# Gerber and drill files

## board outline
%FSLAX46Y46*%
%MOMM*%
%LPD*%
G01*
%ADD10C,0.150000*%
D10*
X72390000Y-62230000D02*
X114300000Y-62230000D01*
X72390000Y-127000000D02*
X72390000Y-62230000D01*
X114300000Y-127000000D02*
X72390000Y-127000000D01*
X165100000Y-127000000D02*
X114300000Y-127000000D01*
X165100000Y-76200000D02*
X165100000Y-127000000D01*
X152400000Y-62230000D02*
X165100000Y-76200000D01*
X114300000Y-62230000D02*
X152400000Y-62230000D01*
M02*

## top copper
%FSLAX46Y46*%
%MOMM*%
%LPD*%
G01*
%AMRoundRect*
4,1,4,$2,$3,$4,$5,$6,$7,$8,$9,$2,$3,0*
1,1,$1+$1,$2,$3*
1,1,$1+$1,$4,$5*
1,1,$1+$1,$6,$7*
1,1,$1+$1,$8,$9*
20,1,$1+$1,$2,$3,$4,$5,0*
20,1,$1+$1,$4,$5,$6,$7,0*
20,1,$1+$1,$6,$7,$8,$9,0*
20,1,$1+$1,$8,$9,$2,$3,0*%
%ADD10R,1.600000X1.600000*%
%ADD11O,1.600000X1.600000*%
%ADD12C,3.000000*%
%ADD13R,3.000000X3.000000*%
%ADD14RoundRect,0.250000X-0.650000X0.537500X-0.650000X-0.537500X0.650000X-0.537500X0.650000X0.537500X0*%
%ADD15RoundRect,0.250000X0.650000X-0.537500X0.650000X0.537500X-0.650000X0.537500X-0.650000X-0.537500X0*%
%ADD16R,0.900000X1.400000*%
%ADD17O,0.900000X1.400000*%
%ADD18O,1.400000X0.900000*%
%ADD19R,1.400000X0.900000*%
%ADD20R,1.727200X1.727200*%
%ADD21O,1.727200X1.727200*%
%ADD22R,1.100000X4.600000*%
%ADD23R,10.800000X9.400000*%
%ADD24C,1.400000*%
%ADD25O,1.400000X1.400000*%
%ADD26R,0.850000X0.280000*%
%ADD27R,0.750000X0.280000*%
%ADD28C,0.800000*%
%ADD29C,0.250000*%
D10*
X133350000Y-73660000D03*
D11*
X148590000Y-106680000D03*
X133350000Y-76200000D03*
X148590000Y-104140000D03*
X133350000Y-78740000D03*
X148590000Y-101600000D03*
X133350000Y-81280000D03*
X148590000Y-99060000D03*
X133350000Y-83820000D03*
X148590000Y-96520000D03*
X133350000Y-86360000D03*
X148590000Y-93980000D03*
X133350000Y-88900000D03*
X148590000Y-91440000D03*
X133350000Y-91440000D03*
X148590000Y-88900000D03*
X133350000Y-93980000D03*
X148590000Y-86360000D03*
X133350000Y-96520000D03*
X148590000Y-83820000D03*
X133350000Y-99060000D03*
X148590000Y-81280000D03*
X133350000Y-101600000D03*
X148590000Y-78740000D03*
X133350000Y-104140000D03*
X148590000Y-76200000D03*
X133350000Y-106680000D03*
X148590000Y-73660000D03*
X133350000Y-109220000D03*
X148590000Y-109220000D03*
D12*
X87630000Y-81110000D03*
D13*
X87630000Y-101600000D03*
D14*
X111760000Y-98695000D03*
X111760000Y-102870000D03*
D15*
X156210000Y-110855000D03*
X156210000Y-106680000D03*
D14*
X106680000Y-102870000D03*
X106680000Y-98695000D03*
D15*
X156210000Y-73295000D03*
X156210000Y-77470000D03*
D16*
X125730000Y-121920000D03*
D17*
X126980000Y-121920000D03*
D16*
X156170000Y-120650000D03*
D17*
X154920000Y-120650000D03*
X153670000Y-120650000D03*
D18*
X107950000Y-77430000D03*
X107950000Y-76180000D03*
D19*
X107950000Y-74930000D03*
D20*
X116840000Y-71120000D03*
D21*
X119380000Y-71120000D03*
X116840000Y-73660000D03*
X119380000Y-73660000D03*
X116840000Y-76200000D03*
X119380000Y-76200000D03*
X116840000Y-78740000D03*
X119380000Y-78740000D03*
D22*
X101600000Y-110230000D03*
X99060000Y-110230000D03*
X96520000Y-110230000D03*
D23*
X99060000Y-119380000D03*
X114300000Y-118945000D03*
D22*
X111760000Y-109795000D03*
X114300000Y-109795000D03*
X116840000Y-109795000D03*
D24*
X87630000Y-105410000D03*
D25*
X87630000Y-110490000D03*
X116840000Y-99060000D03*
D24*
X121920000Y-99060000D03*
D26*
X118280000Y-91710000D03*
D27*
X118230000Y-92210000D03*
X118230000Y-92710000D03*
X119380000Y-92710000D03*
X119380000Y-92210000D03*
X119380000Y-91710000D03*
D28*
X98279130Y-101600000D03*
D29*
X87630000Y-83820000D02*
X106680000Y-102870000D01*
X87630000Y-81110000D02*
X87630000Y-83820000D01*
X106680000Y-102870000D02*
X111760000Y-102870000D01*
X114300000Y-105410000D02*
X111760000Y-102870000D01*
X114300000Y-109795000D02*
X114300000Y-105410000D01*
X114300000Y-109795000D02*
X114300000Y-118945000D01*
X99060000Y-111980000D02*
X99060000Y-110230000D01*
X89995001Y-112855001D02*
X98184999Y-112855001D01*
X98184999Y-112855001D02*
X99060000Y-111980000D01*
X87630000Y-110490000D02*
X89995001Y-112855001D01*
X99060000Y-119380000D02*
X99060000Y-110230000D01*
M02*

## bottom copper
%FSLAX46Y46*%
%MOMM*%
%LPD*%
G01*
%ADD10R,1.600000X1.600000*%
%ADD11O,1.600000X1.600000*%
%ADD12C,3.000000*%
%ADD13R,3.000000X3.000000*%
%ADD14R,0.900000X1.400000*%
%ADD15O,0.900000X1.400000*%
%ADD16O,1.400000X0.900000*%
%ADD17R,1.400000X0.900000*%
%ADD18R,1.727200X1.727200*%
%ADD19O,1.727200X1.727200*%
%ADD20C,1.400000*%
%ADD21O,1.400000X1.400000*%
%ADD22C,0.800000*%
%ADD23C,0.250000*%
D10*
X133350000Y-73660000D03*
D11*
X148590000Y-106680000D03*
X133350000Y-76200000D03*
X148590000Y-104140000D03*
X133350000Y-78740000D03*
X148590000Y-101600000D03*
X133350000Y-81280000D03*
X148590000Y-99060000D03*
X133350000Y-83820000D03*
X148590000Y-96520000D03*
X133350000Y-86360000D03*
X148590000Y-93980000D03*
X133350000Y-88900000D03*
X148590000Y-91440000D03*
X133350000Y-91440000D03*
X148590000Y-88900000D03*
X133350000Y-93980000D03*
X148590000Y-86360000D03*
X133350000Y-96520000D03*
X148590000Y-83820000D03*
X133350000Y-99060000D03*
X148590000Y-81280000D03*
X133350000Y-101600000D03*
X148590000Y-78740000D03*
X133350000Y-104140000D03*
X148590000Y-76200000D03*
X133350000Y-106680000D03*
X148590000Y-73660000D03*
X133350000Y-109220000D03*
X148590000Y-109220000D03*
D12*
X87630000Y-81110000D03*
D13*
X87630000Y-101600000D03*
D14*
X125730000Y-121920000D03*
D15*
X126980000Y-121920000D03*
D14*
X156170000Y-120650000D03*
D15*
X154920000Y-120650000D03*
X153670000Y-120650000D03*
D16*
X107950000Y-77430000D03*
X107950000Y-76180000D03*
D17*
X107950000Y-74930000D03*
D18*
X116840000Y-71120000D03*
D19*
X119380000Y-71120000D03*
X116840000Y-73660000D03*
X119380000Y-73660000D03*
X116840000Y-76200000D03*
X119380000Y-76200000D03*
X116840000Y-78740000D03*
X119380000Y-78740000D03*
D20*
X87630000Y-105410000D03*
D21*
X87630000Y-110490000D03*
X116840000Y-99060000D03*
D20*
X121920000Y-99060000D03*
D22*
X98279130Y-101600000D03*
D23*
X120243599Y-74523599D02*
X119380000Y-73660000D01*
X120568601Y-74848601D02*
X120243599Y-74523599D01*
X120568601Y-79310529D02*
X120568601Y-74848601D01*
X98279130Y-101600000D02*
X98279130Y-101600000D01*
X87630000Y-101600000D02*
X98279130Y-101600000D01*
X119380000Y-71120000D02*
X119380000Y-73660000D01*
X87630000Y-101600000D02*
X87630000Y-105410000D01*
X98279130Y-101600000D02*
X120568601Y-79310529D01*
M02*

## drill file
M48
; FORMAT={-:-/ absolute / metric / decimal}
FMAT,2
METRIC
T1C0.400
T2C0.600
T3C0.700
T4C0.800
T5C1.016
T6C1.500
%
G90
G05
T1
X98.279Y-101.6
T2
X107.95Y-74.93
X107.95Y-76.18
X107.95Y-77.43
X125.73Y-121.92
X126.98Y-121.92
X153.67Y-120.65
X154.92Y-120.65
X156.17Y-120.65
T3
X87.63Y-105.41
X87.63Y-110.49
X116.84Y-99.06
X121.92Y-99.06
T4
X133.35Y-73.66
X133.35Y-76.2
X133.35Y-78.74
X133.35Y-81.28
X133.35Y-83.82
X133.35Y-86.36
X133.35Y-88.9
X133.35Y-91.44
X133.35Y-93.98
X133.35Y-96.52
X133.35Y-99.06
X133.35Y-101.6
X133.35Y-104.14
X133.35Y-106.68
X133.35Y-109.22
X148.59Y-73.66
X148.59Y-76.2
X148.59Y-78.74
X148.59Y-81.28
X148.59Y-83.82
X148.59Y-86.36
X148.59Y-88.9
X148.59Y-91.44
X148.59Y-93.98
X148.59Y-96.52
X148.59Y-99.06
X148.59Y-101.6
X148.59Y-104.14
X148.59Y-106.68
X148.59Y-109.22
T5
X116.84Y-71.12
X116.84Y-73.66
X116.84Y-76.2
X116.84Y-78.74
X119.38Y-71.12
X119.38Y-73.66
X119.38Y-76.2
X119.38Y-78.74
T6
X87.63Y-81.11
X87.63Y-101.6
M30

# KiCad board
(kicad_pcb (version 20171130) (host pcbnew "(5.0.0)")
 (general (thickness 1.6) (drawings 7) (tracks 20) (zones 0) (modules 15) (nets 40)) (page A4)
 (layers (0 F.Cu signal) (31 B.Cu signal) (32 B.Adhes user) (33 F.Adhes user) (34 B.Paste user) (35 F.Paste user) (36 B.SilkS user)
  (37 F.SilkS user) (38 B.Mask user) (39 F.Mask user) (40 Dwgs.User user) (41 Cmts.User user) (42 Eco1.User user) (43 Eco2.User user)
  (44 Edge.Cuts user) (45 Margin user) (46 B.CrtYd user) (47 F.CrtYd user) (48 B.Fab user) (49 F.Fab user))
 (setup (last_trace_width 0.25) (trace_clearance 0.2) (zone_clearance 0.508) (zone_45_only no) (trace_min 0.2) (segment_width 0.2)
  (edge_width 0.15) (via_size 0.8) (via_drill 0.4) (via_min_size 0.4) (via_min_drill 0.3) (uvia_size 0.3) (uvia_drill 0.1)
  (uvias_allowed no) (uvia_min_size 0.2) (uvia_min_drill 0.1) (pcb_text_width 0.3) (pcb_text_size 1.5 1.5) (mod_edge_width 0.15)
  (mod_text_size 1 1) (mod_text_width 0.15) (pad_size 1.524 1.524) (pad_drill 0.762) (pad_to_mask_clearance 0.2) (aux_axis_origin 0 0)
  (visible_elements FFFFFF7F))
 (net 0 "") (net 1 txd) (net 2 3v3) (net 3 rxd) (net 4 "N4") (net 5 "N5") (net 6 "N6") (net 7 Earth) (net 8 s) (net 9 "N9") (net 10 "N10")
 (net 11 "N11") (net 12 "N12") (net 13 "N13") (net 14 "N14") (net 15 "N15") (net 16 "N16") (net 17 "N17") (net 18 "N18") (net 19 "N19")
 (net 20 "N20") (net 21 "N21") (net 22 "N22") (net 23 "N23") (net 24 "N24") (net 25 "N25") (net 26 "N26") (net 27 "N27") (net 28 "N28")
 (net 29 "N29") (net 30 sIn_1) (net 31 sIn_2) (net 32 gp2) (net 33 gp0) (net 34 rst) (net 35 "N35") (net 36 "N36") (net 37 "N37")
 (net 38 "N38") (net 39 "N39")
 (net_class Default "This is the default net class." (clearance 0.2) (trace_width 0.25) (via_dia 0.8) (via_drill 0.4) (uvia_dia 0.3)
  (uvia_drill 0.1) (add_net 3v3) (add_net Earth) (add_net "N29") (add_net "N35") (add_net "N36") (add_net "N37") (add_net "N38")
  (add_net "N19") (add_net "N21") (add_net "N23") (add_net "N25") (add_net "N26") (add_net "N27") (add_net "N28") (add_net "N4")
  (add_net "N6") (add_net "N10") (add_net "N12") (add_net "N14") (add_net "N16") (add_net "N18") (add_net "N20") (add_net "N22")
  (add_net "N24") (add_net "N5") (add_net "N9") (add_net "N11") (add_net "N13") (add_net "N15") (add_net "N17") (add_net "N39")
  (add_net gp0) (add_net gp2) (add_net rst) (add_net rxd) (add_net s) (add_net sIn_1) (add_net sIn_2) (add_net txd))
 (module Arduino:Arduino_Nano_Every (layer F.Cu) (at 133.35 73.66)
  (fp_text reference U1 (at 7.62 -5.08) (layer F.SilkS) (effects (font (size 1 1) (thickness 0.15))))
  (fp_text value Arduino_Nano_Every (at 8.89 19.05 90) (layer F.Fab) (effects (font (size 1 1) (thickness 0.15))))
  (pad 1 thru_hole rect (at 0 0) (size 1.6 1.6) (drill 0.8) (layers *.Cu *.Mask) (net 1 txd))
  (pad 17 thru_hole oval (at 15.24 33.02) (size 1.6 1.6) (drill 0.8) (layers *.Cu *.Mask) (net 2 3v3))
  (pad 2 thru_hole oval (at 0 2.54) (size 1.6 1.6) (drill 0.8) (layers *.Cu *.Mask) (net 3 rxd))
  (pad 18 thru_hole oval (at 15.24 30.48) (size 1.6 1.6) (drill 0.8) (layers *.Cu *.Mask) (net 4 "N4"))
  (pad 3 thru_hole oval (at 0 5.08) (size 1.6 1.6) (drill 0.8) (layers *.Cu *.Mask) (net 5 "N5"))
  (pad 19 thru_hole oval (at 15.24 27.94) (size 1.6 1.6) (drill 0.8) (layers *.Cu *.Mask) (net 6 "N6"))
  (pad 4 thru_hole oval (at 0 7.62) (size 1.6 1.6) (drill 0.8) (layers *.Cu *.Mask) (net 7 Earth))
  (pad 20 thru_hole oval (at 15.24 25.4) (size 1.6 1.6) (drill 0.8) (layers *.Cu *.Mask) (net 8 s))
  (pad 5 thru_hole oval (at 0 10.16) (size 1.6 1.6) (drill 0.8) (layers *.Cu *.Mask) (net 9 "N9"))
  (pad 21 thru_hole oval (at 15.24 22.86) (size 1.6 1.6) (drill 0.8) (layers *.Cu *.Mask) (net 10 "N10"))
  (pad 6 thru_hole oval (at 0 12.7) (size 1.6 1.6) (drill 0.8) (layers *.Cu *.Mask) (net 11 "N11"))
  (pad 22 thru_hole oval (at 15.24 20.32) (size 1.6 1.6) (drill 0.8) (layers *.Cu *.Mask) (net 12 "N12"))
  (pad 7 thru_hole oval (at 0 15.24) (size 1.6 1.6) (drill 0.8) (layers *.Cu *.Mask) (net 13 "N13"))
  (pad 23 thru_hole oval (at 15.24 17.78) (size 1.6 1.6) (drill 0.8) (layers *.Cu *.Mask) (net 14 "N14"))
  (pad 8 thru_hole oval (at 0 17.78) (size 1.6 1.6) (drill 0.8) (layers *.Cu *.Mask) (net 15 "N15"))
  (pad 24 thru_hole oval (at 15.24 15.24) (size 1.6 1.6) (drill 0.8) (layers *.Cu *.Mask) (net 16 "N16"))
  (pad 9 thru_hole oval (at 0 20.32) (size 1.6 1.6) (drill 0.8) (layers *.Cu *.Mask) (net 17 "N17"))
  (pad 25 thru_hole oval (at 15.24 12.7) (size 1.6 1.6) (drill 0.8) (layers *.Cu *.Mask) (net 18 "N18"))
  (pad 10 thru_hole oval (at 0 22.86) (size 1.6 1.6) (drill 0.8) (layers *.Cu *.Mask) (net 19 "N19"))
  (pad 26 thru_hole oval (at 15.24 10.16) (size 1.6 1.6) (drill 0.8) (layers *.Cu *.Mask) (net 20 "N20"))
  (pad 11 thru_hole oval (at 0 25.4) (size 1.6 1.6) (drill 0.8) (layers *.Cu *.Mask) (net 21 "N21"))
  (pad 27 thru_hole oval (at 15.24 7.62) (size 1.6 1.6) (drill 0.8) (layers *.Cu *.Mask) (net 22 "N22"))
  (pad 12 thru_hole oval (at 0 27.94) (size 1.6 1.6) (drill 0.8) (layers *.Cu *.Mask) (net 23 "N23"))
  (pad 28 thru_hole oval (at 15.24 5.08) (size 1.6 1.6) (drill 0.8) (layers *.Cu *.Mask) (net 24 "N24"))
  (pad 13 thru_hole oval (at 0 30.48) (size 1.6 1.6) (drill 0.8) (layers *.Cu *.Mask) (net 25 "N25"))
  (pad 29 thru_hole oval (at 15.24 2.54) (size 1.6 1.6) (drill 0.8) (layers *.Cu *.Mask) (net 7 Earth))
  (pad 14 thru_hole oval (at 0 33.02) (size 1.6 1.6) (drill 0.8) (layers *.Cu *.Mask) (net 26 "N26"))
  (pad 30 thru_hole oval (at 15.24 0) (size 1.6 1.6) (drill 0.8) (layers *.Cu *.Mask) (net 2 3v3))
  (pad 15 thru_hole oval (at 0 35.56) (size 1.6 1.6) (drill 0.8) (layers *.Cu *.Mask) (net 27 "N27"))
  (pad 16 thru_hole oval (at 15.24 35.56) (size 1.6 1.6) (drill 0.8) (layers *.Cu *.Mask) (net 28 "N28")))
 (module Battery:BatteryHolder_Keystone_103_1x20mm (layer F.Cu) (at 87.63 101.6 90)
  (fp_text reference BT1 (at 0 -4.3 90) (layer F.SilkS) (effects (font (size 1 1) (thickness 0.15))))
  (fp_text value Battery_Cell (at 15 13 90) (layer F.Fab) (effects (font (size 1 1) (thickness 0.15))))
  (pad 2 thru_hole circle (at 20.49 0 90) (size 3 3) (drill 1.5) (layers *.Cu *.Mask) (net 7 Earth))
  (pad 1 thru_hole rect (at 0 0 90) (size 3 3) (drill 1.5) (layers *.Cu *.Mask) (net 2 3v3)))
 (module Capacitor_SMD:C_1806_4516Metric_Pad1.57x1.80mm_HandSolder (layer F.Cu) (at 111.76 100.7825 270)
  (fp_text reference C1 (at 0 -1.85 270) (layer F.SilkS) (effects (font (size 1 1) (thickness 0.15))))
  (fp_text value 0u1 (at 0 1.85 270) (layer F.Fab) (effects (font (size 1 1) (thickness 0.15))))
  (pad 1 smd roundrect (at -2.0875 0 270) (size 1.575 1.8) (layers F.Cu F.Paste F.Mask) (roundrect_rratio 0.15873) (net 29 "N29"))
  (pad 2 smd roundrect (at 2.0875 0 270) (size 1.575 1.8) (layers F.Cu F.Paste F.Mask) (roundrect_rratio 0.15873) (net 7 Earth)))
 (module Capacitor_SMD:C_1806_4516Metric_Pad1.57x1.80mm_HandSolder (layer F.Cu) (at 156.21 108.7675 90)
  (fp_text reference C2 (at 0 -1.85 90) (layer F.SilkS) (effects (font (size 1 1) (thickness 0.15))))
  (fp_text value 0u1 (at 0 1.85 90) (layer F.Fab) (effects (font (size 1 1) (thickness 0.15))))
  (pad 1 smd roundrect (at -2.0875 0 90) (size 1.575 1.8) (layers F.Cu F.Paste F.Mask) (roundrect_rratio 0.15873) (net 7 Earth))
  (pad 2 smd roundrect (at 2.0875 0 90) (size 1.575 1.8) (layers F.Cu F.Paste F.Mask) (roundrect_rratio 0.15873) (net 2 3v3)))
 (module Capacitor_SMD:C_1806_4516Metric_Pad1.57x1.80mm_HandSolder (layer F.Cu) (at 106.68 100.7825 270)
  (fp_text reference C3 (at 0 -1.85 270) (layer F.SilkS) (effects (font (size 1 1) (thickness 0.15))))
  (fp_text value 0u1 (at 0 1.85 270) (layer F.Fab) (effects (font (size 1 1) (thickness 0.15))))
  (pad 2 smd roundrect (at 2.0875 0 270) (size 1.575 1.8) (layers F.Cu F.Paste F.Mask) (roundrect_rratio 0.15873) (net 7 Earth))
  (pad 1 smd roundrect (at -2.0875 0 270) (size 1.575 1.8) (layers F.Cu F.Paste F.Mask) (roundrect_rratio 0.15873) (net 2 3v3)))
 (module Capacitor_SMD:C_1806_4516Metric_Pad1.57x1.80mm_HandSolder (layer F.Cu) (at 156.21 75.3825 90)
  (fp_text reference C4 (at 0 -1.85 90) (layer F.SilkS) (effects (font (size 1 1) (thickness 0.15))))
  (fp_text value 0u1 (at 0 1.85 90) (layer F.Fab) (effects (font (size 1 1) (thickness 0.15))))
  (pad 2 smd roundrect (at 2.0875 0 90) (size 1.575 1.8) (layers F.Cu F.Paste F.Mask) (roundrect_rratio 0.15873) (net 2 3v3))
  (pad 1 smd roundrect (at -2.0875 0 90) (size 1.575 1.8) (layers F.Cu F.Paste F.Mask) (roundrect_rratio 0.15873) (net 7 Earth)))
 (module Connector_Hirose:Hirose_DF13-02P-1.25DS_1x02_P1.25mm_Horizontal (layer F.Cu) (at 125.73 121.92)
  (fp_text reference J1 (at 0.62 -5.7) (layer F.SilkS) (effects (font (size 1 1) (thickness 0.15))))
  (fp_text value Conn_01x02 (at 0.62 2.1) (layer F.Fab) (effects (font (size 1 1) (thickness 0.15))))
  (pad 1 thru_hole rect (at 0 0) (size 0.9 1.4) (drill 0.6) (layers *.Cu *.Mask) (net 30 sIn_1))
  (pad 2 thru_hole oval (at 1.25 0) (size 0.9 1.4) (drill 0.6) (layers *.Cu *.Mask) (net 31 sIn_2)))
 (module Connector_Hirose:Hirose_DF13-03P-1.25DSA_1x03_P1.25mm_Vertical (layer F.Cu) (at 156.17 120.65 180)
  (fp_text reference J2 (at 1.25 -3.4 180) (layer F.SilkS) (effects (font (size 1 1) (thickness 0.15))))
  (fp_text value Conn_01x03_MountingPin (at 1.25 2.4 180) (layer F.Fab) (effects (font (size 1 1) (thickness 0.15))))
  (pad 1 thru_hole rect (at 0 0 180) (size 0.9 1.4) (drill 0.6) (layers *.Cu *.Mask) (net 8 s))
  (pad 2 thru_hole oval (at 1.25 0 180) (size 0.9 1.4) (drill 0.6) (layers *.Cu *.Mask) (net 2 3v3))
  (pad 3 thru_hole oval (at 2.5 0 180) (size 0.9 1.4) (drill 0.6) (layers *.Cu *.Mask) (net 7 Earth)))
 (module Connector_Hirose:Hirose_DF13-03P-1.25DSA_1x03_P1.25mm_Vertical (layer F.Cu) (at 107.95 74.93 270)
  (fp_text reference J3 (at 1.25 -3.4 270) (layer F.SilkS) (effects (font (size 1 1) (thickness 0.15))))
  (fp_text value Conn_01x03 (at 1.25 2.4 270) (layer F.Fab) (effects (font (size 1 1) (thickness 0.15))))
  (pad 3 thru_hole oval (at 2.5 0 270) (size 0.9 1.4) (drill 0.6) (layers *.Cu *.Mask) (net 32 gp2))
  (pad 2 thru_hole oval (at 1.25 0 270) (size 0.9 1.4) (drill 0.6) (layers *.Cu *.Mask) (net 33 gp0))
  (pad 1 thru_hole rect (at 0 0 270) (size 0.9 1.4) (drill 0.6) (layers *.Cu *.Mask) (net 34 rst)))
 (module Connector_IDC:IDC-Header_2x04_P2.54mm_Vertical (layer F.Cu) (at 116.84 71.12)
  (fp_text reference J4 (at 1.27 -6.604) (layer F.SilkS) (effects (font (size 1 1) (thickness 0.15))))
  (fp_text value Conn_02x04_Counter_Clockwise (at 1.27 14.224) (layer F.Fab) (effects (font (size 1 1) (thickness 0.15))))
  (pad 1 thru_hole rect (at 0 0) (size 1.7272 1.7272) (drill 1.016) (layers *.Cu *.Mask) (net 1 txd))
  (pad 2 thru_hole oval (at 2.54 0) (size 1.7272 1.7272) (drill 1.016) (layers *.Cu *.Mask) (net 2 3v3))
  (pad 3 thru_hole oval (at 0 2.54) (size 1.7272 1.7272) (drill 1.016) (layers *.Cu *.Mask) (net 34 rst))
  (pad 4 thru_hole oval (at 2.54 2.54) (size 1.7272 1.7272) (drill 1.016) (layers *.Cu *.Mask) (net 2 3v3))
  (pad 5 thru_hole oval (at 0 5.08) (size 1.7272 1.7272) (drill 1.016) (layers *.Cu *.Mask) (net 3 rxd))
  (pad 6 thru_hole oval (at 2.54 5.08) (size 1.7272 1.7272) (drill 1.016) (layers *.Cu *.Mask) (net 33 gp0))
  (pad 7 thru_hole oval (at 0 7.62) (size 1.7272 1.7272) (drill 1.016) (layers *.Cu *.Mask) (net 32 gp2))
  (pad 8 thru_hole oval (at 2.54 7.62) (size 1.7272 1.7272) (drill 1.016) (layers *.Cu *.Mask) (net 7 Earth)))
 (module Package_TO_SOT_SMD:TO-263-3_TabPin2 (layer F.Cu) (at 99.06 116.005 270)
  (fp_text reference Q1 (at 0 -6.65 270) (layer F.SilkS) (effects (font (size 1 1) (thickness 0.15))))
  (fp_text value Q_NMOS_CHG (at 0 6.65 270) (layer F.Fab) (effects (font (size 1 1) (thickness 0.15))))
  (pad 1 smd rect (at -5.775 -2.54 270) (size 4.6 1.1) (layers F.Cu F.Paste F.Mask) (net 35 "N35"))
  (pad 2 smd rect (at -5.775 0 270) (size 4.6 1.1) (layers F.Cu F.Paste F.Mask) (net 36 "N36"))
  (pad 3 smd rect (at -5.775 2.54 270) (size 4.6 1.1) (layers F.Cu F.Paste F.Mask) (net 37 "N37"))
  (pad 2 smd rect (at 3.375 0 270) (size 9.4 10.8) (layers F.Cu F.Mask) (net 36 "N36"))
  (pad "" smd rect (at 5.8 2.775 270) (size 4.55 5.25) (layers F.Paste))
  (pad "" smd rect (at 0.95 -2.775 270) (size 4.55 5.25) (layers F.Paste))
  (pad "" smd rect (at 5.8 -2.775 270) (size 4.55 5.25) (layers F.Paste))
  (pad "" smd rect (at 0.95 2.775 270) (size 4.55 5.25) (layers F.Paste)))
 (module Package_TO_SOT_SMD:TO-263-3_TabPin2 (layer F.Cu) (at 114.3 115.57 270)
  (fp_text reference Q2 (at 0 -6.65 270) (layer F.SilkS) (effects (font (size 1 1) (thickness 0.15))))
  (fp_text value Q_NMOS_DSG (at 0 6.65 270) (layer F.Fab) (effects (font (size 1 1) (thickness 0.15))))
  (pad "" smd rect (at 0.95 2.775 270) (size 4.55 5.25) (layers F.Paste))
  (pad "" smd rect (at 5.8 -2.775 270) (size 4.55 5.25) (layers F.Paste))
  (pad "" smd rect (at 0.95 -2.775 270) (size 4.55 5.25) (layers F.Paste))
  (pad "" smd rect (at 5.8 2.775 270) (size 4.55 5.25) (layers F.Paste))
  (pad 2 smd rect (at 3.375 0 270) (size 9.4 10.8) (layers F.Cu F.Mask) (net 7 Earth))
  (pad 3 smd rect (at -5.775 2.54 270) (size 4.6 1.1) (layers F.Cu F.Paste F.Mask) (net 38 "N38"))
  (pad 2 smd rect (at -5.775 0 270) (size 4.6 1.1) (layers F.Cu F.Paste F.Mask) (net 7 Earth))
  (pad 1 smd rect (at -5.775 -2.54 270) (size 4.6 1.1) (layers F.Cu F.Paste F.Mask) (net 35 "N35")))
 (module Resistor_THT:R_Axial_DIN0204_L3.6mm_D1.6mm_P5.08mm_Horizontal (layer F.Cu) (at 87.63 105.41 270)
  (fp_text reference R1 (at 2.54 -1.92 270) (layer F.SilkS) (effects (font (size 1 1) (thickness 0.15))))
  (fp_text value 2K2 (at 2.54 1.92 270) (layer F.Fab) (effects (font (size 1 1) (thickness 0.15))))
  (pad 1 thru_hole circle (at 0 0 270) (size 1.4 1.4) (drill 0.7) (layers *.Cu *.Mask) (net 2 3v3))
  (pad 2 thru_hole oval (at 5.08 0 270) (size 1.4 1.4) (drill 0.7) (layers *.Cu *.Mask) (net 36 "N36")))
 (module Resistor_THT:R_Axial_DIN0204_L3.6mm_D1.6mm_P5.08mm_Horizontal (layer F.Cu) (at 121.92 99.06 180)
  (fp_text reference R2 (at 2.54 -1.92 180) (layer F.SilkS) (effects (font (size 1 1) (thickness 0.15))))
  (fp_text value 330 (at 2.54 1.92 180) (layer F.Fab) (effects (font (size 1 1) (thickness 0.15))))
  (pad 2 thru_hole oval (at 5.08 0 180) (size 1.4 1.4) (drill 0.7) (layers *.Cu *.Mask) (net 29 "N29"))
  (pad 1 thru_hole circle (at 0 0 180) (size 1.4 1.4) (drill 0.7) (layers *.Cu *.Mask) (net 2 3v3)))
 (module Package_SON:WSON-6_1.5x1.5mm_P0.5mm (layer F.Cu) (at 118.805 92.21)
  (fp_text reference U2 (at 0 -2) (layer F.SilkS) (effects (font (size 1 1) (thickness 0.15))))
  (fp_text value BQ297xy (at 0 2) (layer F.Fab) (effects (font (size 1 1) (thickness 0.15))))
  (pad 1 smd rect (at -0.525 -0.5 270) (size 0.28 0.85) (layers F.Cu F.Paste F.Mask) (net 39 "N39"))
  (pad 2 smd rect (at -0.575 0 270) (size 0.28 0.75) (layers F.Cu F.Paste F.Mask) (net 37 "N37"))
  (pad 3 smd rect (at -0.575 0.5 270) (size 0.28 0.75) (layers F.Cu F.Paste F.Mask) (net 38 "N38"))
  (pad 4 smd rect (at 0.575 0.5 270) (size 0.28 0.75) (layers F.Cu F.Paste F.Mask) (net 7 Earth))
  (pad 5 smd rect (at 0.575 0 270) (size 0.28 0.75) (layers F.Cu F.Paste F.Mask) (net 29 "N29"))
  (pad 6 smd rect (at 0.575 -0.5 270) (size 0.28 0.75) (layers F.Cu F.Paste F.Mask) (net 2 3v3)))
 (gr_line (start 72.39 62.23) (end 114.3 62.23) (layer Edge.Cuts) (width 0.15))
 (gr_line (start 72.39 127) (end 72.39 62.23) (layer Edge.Cuts) (width 0.15))
 (gr_line (start 114.3 127) (end 72.39 127) (layer Edge.Cuts) (width 0.15))
 (gr_line (start 165.1 127) (end 114.3 127) (layer Edge.Cuts) (width 0.15))
 (gr_line (start 165.1 76.2) (end 165.1 127) (layer Edge.Cuts) (width 0.15))
 (gr_line (start 152.4 62.23) (end 165.1 76.2) (layer Edge.Cuts) (width 0.15))
 (gr_line (start 114.3 62.23) (end 152.4 62.23) (layer Edge.Cuts) (width 0.15))
 (segment (start 87.63 83.82) (end 106.68 102.87) (width 0.25) (layer F.Cu) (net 7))
 (segment (start 87.63 81.11) (end 87.63 83.82) (width 0.25) (layer F.Cu) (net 7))
 (segment (start 106.68 102.87) (end 111.76 102.87) (width 0.25) (layer F.Cu) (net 7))
 (segment (start 114.3 105.41) (end 111.76 102.87) (width 0.25) (layer F.Cu) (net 7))
 (segment (start 114.3 109.795) (end 114.3 105.41) (width 0.25) (layer F.Cu) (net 7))
 (segment (start 114.3 109.795) (end 114.3 118.945) (width 0.25) (layer F.Cu) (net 7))
 (segment (start 120.243599 74.523599) (end 119.38 73.66) (width 0.25) (layer B.Cu) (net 2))
 (segment (start 120.568601 74.848601) (end 120.243599 74.523599) (width 0.25) (layer B.Cu) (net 2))
 (segment (start 120.568601 79.310529) (end 120.568601 74.848601) (width 0.25) (layer B.Cu) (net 2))
 (segment (start 98.27913 101.6) (end 98.27913 101.6) (width 0.25) (layer B.Cu) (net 2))
 (segment (start 87.63 101.6) (end 98.27913 101.6) (width 0.25) (layer B.Cu) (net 2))
 (segment (start 119.38 71.12) (end 119.38 73.66) (width 0.25) (layer B.Cu) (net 2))
 (segment (start 87.63 101.6) (end 87.63 105.41) (width 0.25) (layer B.Cu) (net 2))
 (segment (start 98.27913 101.6) (end 120.568601 79.310529) (width 0.25) (layer B.Cu) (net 2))
 (via (at 98.27913 101.6) (size 0.8) (drill 0.4) (layers F.Cu B.Cu) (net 2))
 (segment (start 99.06 111.98) (end 99.06 110.23) (width 0.25) (layer F.Cu) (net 36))
 (segment (start 89.995001 112.855001) (end 98.184999 112.855001) (width 0.25) (layer F.Cu) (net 36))
 (segment (start 98.184999 112.855001) (end 99.06 111.98) (width 0.25) (layer F.Cu) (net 36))
 (segment (start 87.63 110.49) (end 89.995001 112.855001) (width 0.25) (layer F.Cu) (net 36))
 (segment (start 99.06 119.38) (end 99.06 110.23) (width 0.25) (layer F.Cu) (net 36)))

